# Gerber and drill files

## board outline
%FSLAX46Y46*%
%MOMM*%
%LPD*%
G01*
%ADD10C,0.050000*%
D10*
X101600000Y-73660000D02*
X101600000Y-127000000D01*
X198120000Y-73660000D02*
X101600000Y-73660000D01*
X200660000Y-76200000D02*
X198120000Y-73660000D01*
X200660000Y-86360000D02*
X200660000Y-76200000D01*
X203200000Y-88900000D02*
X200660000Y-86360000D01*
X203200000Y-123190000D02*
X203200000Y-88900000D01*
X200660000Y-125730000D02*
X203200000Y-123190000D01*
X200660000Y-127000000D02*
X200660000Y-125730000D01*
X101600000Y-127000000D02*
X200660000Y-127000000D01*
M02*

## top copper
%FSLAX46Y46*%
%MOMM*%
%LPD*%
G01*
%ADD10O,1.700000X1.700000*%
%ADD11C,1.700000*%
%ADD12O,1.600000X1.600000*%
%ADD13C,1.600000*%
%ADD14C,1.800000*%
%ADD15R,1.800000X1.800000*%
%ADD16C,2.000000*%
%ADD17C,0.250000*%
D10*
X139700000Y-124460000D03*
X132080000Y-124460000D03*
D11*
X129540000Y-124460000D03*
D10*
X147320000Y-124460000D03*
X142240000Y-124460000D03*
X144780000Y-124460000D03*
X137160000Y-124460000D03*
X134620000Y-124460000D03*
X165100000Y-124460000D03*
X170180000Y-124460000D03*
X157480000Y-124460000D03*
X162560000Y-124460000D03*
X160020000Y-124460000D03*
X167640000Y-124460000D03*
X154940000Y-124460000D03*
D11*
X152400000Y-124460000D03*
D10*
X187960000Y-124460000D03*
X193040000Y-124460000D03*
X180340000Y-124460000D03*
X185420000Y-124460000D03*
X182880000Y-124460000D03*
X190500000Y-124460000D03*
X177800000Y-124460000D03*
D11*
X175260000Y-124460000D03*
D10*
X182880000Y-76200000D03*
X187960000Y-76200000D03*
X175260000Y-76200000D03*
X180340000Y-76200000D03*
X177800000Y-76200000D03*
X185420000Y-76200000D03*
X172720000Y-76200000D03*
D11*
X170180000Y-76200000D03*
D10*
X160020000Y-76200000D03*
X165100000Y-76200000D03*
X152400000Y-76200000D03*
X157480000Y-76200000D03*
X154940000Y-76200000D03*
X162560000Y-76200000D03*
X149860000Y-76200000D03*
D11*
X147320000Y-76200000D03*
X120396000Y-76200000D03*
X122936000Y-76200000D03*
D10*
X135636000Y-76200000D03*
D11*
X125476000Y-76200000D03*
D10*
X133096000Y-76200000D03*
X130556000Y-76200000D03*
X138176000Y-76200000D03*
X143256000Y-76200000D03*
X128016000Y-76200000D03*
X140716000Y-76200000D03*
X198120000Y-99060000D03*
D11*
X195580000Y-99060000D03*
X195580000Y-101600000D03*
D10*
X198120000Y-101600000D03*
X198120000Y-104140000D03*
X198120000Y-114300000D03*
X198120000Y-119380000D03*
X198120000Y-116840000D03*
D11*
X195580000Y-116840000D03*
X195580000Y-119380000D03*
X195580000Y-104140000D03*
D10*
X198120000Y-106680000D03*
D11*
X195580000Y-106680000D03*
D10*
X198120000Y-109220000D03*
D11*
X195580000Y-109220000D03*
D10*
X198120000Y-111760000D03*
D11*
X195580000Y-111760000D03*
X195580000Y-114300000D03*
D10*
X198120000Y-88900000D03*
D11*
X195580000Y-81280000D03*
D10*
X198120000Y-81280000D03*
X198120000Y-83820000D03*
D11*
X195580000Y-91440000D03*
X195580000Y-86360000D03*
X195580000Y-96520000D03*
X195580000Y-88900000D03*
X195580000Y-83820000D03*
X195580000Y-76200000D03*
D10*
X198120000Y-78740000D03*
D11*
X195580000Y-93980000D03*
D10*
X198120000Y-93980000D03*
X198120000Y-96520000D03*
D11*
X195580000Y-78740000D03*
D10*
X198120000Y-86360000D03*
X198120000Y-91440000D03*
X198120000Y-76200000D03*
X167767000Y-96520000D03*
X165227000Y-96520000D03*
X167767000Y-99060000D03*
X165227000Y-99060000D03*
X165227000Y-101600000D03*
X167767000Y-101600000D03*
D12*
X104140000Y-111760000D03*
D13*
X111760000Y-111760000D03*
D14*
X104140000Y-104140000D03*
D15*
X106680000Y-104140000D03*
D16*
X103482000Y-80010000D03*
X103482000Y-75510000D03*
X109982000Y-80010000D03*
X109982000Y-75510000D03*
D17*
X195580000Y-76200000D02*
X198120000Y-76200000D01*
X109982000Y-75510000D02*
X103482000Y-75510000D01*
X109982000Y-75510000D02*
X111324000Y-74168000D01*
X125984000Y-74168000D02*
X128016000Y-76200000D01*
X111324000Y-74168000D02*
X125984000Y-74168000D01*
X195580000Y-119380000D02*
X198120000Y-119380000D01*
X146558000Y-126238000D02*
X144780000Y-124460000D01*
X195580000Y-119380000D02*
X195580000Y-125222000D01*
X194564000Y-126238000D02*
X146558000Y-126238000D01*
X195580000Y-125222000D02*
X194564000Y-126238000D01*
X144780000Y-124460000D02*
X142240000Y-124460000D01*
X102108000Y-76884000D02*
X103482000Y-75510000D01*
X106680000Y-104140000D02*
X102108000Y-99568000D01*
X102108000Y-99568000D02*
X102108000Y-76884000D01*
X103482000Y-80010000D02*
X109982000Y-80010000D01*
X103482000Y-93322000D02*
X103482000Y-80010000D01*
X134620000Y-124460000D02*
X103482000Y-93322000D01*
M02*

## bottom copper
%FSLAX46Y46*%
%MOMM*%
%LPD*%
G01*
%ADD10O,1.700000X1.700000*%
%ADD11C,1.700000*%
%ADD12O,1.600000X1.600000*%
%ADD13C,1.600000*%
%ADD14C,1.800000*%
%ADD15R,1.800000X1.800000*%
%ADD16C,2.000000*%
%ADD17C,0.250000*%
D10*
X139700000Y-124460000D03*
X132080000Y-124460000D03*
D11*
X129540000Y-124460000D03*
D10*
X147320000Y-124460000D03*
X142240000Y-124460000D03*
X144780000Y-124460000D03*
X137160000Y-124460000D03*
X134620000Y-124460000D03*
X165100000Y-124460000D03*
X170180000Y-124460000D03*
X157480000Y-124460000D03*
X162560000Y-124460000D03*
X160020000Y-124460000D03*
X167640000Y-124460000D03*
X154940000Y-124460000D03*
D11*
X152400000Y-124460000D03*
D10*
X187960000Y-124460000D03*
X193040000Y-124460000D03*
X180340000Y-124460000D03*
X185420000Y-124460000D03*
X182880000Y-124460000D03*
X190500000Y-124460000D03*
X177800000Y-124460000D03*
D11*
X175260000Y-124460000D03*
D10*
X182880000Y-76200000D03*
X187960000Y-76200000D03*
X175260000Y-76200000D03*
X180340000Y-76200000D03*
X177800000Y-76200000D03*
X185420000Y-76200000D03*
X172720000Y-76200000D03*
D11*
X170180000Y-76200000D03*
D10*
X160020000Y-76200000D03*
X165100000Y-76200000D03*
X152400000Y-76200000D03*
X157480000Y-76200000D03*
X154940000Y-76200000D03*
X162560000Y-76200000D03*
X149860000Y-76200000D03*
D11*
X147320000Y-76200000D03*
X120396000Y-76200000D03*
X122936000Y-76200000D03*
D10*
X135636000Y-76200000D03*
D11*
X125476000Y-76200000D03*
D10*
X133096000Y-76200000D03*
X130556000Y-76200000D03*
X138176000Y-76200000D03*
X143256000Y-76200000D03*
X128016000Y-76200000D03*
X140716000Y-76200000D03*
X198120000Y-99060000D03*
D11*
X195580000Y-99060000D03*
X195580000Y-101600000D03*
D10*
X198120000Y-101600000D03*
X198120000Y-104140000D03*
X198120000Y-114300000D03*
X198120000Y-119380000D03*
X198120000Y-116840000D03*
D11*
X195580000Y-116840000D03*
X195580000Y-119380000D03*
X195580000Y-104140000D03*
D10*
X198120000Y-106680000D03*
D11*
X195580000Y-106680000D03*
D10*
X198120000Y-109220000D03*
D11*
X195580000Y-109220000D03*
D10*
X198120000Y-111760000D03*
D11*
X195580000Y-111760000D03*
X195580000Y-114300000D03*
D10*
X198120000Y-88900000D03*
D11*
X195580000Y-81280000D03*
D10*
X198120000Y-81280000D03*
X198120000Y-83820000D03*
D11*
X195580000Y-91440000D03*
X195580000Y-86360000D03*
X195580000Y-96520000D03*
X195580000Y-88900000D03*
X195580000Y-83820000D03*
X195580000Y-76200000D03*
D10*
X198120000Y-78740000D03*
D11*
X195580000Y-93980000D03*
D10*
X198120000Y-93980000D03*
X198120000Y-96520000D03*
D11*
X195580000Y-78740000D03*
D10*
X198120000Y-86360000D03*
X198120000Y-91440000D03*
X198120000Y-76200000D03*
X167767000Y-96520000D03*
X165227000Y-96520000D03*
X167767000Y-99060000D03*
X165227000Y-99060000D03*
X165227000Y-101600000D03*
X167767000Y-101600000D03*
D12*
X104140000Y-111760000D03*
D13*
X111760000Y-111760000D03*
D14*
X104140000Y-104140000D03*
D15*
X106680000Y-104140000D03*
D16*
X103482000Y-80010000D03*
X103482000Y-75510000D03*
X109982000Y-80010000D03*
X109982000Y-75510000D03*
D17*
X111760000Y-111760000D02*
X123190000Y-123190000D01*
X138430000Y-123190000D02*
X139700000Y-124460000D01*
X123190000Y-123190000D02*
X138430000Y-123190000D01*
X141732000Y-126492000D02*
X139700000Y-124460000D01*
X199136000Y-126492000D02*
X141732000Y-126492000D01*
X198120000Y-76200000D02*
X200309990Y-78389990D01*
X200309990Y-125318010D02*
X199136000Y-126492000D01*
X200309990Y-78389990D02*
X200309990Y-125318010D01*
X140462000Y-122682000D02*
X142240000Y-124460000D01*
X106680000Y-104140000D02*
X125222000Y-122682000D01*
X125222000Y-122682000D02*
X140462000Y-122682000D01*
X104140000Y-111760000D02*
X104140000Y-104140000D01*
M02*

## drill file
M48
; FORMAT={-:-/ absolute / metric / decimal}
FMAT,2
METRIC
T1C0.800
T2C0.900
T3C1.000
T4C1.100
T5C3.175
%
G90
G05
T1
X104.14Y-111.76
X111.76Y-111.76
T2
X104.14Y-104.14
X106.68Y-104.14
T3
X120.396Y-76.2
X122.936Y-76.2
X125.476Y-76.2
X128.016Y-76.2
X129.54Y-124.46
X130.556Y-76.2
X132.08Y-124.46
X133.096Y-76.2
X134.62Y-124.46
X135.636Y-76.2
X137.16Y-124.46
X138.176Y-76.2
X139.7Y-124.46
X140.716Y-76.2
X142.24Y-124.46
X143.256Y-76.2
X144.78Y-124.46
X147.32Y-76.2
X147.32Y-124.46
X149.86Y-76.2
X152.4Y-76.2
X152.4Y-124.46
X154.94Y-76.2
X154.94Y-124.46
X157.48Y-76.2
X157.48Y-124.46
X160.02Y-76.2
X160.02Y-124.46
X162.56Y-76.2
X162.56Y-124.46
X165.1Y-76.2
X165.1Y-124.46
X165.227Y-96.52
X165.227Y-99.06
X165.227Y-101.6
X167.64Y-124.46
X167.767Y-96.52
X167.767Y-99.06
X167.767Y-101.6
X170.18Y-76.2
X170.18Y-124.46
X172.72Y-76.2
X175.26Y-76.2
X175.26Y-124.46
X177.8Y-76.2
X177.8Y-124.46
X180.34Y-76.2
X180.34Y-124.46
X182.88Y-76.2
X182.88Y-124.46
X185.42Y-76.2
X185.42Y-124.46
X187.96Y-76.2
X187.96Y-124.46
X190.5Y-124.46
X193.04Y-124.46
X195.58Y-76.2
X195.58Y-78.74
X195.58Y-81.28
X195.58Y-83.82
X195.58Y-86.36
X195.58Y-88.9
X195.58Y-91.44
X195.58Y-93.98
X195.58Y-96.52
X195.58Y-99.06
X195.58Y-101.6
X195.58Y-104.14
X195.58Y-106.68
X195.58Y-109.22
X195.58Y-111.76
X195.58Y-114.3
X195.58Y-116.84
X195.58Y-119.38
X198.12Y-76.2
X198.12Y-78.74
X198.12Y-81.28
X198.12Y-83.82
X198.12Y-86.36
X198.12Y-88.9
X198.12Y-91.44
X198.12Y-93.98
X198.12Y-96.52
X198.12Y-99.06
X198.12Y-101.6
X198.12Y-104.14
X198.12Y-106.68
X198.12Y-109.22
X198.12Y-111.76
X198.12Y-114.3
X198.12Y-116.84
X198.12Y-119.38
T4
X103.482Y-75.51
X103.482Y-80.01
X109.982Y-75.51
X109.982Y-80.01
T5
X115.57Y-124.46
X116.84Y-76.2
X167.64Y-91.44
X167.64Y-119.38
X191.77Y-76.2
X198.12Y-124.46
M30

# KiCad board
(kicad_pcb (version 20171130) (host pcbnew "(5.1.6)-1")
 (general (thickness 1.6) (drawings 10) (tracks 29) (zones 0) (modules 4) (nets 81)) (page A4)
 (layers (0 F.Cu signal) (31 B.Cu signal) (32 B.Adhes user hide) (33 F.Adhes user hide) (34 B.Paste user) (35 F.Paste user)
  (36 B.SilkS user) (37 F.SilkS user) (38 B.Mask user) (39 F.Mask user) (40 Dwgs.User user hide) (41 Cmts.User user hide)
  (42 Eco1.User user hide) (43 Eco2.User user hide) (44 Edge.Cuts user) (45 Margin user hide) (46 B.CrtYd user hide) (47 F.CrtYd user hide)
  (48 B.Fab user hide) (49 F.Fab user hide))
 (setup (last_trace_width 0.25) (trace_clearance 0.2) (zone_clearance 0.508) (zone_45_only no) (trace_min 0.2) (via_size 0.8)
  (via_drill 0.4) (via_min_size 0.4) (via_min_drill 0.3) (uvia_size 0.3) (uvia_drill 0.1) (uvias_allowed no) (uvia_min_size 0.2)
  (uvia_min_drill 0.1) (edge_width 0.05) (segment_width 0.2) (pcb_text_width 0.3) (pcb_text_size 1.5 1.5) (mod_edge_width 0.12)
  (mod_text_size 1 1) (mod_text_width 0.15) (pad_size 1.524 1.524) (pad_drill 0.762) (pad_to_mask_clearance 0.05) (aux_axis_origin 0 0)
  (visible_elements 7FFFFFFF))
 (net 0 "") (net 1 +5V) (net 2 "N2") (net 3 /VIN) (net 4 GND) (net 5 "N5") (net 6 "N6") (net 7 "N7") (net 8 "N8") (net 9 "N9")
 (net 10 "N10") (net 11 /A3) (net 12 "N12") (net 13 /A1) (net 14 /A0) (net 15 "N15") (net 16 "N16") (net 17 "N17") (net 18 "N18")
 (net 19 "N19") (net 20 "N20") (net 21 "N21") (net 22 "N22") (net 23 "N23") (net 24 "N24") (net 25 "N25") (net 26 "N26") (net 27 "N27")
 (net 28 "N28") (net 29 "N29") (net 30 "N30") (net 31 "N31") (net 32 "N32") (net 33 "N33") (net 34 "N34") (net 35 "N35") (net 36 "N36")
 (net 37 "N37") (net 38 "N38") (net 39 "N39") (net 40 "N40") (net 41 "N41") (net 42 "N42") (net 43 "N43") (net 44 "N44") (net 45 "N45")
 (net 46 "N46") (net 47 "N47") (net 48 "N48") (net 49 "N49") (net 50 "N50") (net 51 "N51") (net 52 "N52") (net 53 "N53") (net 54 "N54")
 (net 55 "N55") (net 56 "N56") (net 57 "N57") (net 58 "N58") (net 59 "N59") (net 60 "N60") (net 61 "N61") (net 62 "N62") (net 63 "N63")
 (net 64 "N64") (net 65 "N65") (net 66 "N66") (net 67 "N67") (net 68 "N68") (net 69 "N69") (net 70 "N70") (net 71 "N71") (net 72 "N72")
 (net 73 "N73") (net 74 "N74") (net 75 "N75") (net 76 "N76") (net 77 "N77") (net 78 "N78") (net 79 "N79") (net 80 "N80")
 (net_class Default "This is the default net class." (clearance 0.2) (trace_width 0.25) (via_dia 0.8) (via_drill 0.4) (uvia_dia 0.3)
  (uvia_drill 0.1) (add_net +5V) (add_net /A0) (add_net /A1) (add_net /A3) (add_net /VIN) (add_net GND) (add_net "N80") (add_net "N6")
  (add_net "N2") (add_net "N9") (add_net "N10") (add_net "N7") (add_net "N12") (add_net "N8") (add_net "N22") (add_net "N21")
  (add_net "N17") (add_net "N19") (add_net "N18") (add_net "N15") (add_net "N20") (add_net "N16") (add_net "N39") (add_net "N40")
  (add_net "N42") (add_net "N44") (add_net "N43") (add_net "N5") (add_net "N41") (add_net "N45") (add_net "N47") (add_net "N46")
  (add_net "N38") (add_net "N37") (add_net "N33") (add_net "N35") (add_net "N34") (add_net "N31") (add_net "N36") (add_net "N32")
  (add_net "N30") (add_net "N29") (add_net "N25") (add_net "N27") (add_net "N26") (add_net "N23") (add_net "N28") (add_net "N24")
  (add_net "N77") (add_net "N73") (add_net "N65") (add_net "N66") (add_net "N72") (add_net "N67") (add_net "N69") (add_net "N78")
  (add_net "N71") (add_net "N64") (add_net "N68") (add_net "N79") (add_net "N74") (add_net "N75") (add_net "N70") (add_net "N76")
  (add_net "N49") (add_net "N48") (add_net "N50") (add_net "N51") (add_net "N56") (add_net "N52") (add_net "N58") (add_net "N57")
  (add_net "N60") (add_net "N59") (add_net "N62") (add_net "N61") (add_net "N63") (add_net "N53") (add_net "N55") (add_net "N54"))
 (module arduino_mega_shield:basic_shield (layer F.Cu) (at 101.6 127)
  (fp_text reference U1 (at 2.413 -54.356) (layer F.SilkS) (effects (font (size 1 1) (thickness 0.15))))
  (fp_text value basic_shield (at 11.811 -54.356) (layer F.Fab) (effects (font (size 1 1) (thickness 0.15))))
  (pad 4 thru_hole oval (at 38.1 -2.54 90) (size 1.7 1.7) (drill 1) (layers *.Cu *.Mask) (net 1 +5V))
  (pad 1 thru_hole oval (at 30.48 -2.54 90) (size 1.7 1.7) (drill 1) (layers *.Cu *.Mask) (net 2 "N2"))
  (pad "" thru_hole circle (at 27.94 -2.54 90) (size 1.7 1.7) (drill 1) (layers *.Cu *.Mask))
  (pad 7 thru_hole oval (at 45.72 -2.54 90) (size 1.7 1.7) (drill 1) (layers *.Cu *.Mask) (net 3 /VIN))
  (pad 5 thru_hole oval (at 40.64 -2.54 90) (size 1.7 1.7) (drill 1) (layers *.Cu *.Mask) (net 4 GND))
  (pad 6 thru_hole oval (at 43.18 -2.54 90) (size 1.7 1.7) (drill 1) (layers *.Cu *.Mask) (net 4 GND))
  (pad 3 thru_hole oval (at 35.56 -2.54 90) (size 1.7 1.7) (drill 1) (layers *.Cu *.Mask) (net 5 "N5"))
  (pad 2 thru_hole oval (at 33.02 -2.54 90) (size 1.7 1.7) (drill 1) (layers *.Cu *.Mask B.SilkS) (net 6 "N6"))
  (pad 13 thru_hole oval (at 63.5 -2.54 90) (size 1.7 1.7) (drill 1) (layers *.Cu *.Mask) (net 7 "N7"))
  (pad 15 thru_hole oval (at 68.58 -2.54 90) (size 1.7 1.7) (drill 1) (layers *.Cu *.Mask) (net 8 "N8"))
  (pad 10 thru_hole oval (at 55.88 -2.54 90) (size 1.7 1.7) (drill 1) (layers *.Cu *.Mask) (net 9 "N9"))
  (pad 12 thru_hole oval (at 60.96 -2.54 90) (size 1.7 1.7) (drill 1) (layers *.Cu *.Mask) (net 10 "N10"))
  (pad 11 thru_hole oval (at 58.42 -2.54 90) (size 1.7 1.7) (drill 1) (layers *.Cu *.Mask) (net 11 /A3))
  (pad 14 thru_hole oval (at 66.04 -2.54 90) (size 1.7 1.7) (drill 1) (layers *.Cu *.Mask) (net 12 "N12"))
  (pad 9 thru_hole oval (at 53.34 -2.54 90) (size 1.7 1.7) (drill 1) (layers *.Cu *.Mask) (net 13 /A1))
  (pad 8 thru_hole circle (at 50.8 -2.54 90) (size 1.7 1.7) (drill 1) (layers *.Cu *.Mask) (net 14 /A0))
  (pad 21 thru_hole oval (at 86.36 -2.54 90) (size 1.7 1.7) (drill 1) (layers *.Cu *.Mask) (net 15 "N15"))
  (pad 23 thru_hole oval (at 91.44 -2.54 90) (size 1.7 1.7) (drill 1) (layers *.Cu *.Mask) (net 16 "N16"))
  (pad 18 thru_hole oval (at 78.74 -2.54 90) (size 1.7 1.7) (drill 1) (layers *.Cu *.Mask) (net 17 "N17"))
  (pad 20 thru_hole oval (at 83.82 -2.54 90) (size 1.7 1.7) (drill 1) (layers *.Cu *.Mask) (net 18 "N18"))
  (pad 19 thru_hole oval (at 81.28 -2.54 90) (size 1.7 1.7) (drill 1) (layers *.Cu *.Mask) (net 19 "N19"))
  (pad 22 thru_hole oval (at 88.9 -2.54 90) (size 1.7 1.7) (drill 1) (layers *.Cu *.Mask) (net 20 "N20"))
  (pad 17 thru_hole oval (at 76.2 -2.54 90) (size 1.7 1.7) (drill 1) (layers *.Cu *.Mask) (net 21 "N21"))
  (pad 16 thru_hole circle (at 73.66 -2.54 90) (size 1.7 1.7) (drill 1) (layers *.Cu *.Mask) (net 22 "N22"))
  (pad 47 thru_hole oval (at 81.28 -50.8 90) (size 1.7 1.7) (drill 1) (layers *.Cu *.Mask) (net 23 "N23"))
  (pad 49 thru_hole oval (at 86.36 -50.8 90) (size 1.7 1.7) (drill 1) (layers *.Cu *.Mask) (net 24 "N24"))
  (pad 44 thru_hole oval (at 73.66 -50.8 90) (size 1.7 1.7) (drill 1) (layers *.Cu *.Mask) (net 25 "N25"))
  (pad 46 thru_hole oval (at 78.74 -50.8 90) (size 1.7 1.7) (drill 1) (layers *.Cu *.Mask) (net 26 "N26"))
  (pad 45 thru_hole oval (at 76.2 -50.8 90) (size 1.7 1.7) (drill 1) (layers *.Cu *.Mask) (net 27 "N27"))
  (pad 48 thru_hole oval (at 83.82 -50.8 90) (size 1.7 1.7) (drill 1) (layers *.Cu *.Mask) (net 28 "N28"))
  (pad 43 thru_hole oval (at 71.12 -50.8 90) (size 1.7 1.7) (drill 1) (layers *.Cu *.Mask) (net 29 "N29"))
  (pad 42 thru_hole circle (at 68.58 -50.8 90) (size 1.7 1.7) (drill 1) (layers *.Cu *.Mask) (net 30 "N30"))
  (pad 39 thru_hole oval (at 58.42 -50.8 90) (size 1.7 1.7) (drill 1) (layers *.Cu *.Mask) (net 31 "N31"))
  (pad 41 thru_hole oval (at 63.5 -50.8 90) (size 1.7 1.7) (drill 1) (layers *.Cu *.Mask) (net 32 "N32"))
  (pad 36 thru_hole oval (at 50.8 -50.8 90) (size 1.7 1.7) (drill 1) (layers *.Cu *.Mask) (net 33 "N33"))
  (pad 38 thru_hole oval (at 55.88 -50.8 90) (size 1.7 1.7) (drill 1) (layers *.Cu *.Mask) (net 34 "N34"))
  (pad 37 thru_hole oval (at 53.34 -50.8 90) (size 1.7 1.7) (drill 1) (layers *.Cu *.Mask) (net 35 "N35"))
  (pad 40 thru_hole oval (at 60.96 -50.8 90) (size 1.7 1.7) (drill 1) (layers *.Cu *.Mask) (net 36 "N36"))
  (pad 35 thru_hole oval (at 48.26 -50.8 90) (size 1.7 1.7) (drill 1) (layers *.Cu *.Mask B.Paste) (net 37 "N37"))
  (pad 34 thru_hole circle (at 45.72 -50.8 90) (size 1.7 1.7) (drill 1) (layers *.Cu *.Mask) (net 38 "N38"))
  (pad 24 thru_hole circle (at 18.796 -50.8 90) (size 1.7 1.7) (drill 1) (layers *.Cu *.Mask) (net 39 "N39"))
  (pad 25 thru_hole circle (at 21.336 -50.8 90) (size 1.7 1.7) (drill 1) (layers *.Cu *.Mask) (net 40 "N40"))
  (pad 30 thru_hole oval (at 34.036 -50.8 90) (size 1.7 1.7) (drill 1) (layers *.Cu *.Mask) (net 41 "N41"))
  (pad 26 thru_hole circle (at 23.876 -50.8 90) (size 1.7 1.7) (drill 1) (layers *.Cu *.Mask) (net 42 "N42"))
  (pad 29 thru_hole oval (at 31.496 -50.8 90) (size 1.7 1.7) (drill 1) (layers *.Cu *.Mask) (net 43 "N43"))
  (pad 28 thru_hole oval (at 28.956 -50.8 90) (size 1.7 1.7) (drill 1) (layers *.Cu *.Mask) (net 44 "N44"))
  (pad 31 thru_hole oval (at 36.576 -50.8 90) (size 1.7 1.7) (drill 1) (layers *.Cu *.Mask) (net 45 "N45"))
  (pad 33 thru_hole oval (at 41.656 -50.8 90) (size 1.7 1.7) (drill 1) (layers *.Cu *.Mask) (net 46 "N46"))
  (pad 27 thru_hole oval (at 26.416 -50.8 90) (size 1.7 1.7) (drill 1) (layers *.Cu *.Mask) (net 4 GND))
  (pad 32 thru_hole oval (at 39.116 -50.8 90) (size 1.7 1.7) (drill 1) (layers *.Cu *.Mask) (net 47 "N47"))
  (pad 69 thru_hole oval (at 96.52 -27.94 90) (size 1.7 1.7) (drill 1) (layers *.Cu *.Mask) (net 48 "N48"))
  (pad 68 thru_hole circle (at 93.98 -27.94 90) (size 1.7 1.7) (drill 1) (layers *.Cu *.Mask) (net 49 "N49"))
  (pad 70 thru_hole circle (at 93.98 -25.4 90) (size 1.7 1.7) (drill 1) (layers *.Cu *.Mask) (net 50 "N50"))
  (pad 71 thru_hole oval (at 96.52 -25.4 90) (size 1.7 1.7) (drill 1) (layers *.Cu *.Mask) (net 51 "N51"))
  (pad 73 thru_hole oval (at 96.52 -22.86 90) (size 1.7 1.7) (drill 1) (layers *.Cu *.Mask) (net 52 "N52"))
  (pad 81 thru_hole oval (at 96.52 -12.7 90) (size 1.7 1.7) (drill 1) (layers *.Cu *.Mask) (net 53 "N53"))
  (pad 85 thru_hole oval (at 96.52 -7.62 90) (size 1.7 1.7) (drill 1) (layers *.Cu *.Mask) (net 4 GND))
  (pad 83 thru_hole oval (at 96.52 -10.16 90) (size 1.7 1.7) (drill 1) (layers *.Cu *.Mask) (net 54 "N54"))
  (pad 82 thru_hole circle (at 93.98 -10.16 90) (size 1.7 1.7) (drill 1) (layers *.Cu *.Mask) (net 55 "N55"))
  (pad 84 thru_hole circle (at 93.98 -7.62 90) (size 1.7 1.7) (drill 1) (layers *.Cu *.Mask) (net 4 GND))
  (pad 72 thru_hole circle (at 93.98 -22.86 90) (size 1.7 1.7) (drill 1) (layers *.Cu *.Mask) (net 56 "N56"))
  (pad 75 thru_hole oval (at 96.52 -20.32 90) (size 1.7 1.7) (drill 1) (layers *.Cu *.Mask) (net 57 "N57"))
  (pad 74 thru_hole circle (at 93.98 -20.32 90) (size 1.7 1.7) (drill 1) (layers *.Cu *.Mask) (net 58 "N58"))
  (pad 77 thru_hole oval (at 96.52 -17.78 90) (size 1.7 1.7) (drill 1) (layers *.Cu *.Mask) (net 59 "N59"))
  (pad 76 thru_hole circle (at 93.98 -17.78 90) (size 1.7 1.7) (drill 1) (layers *.Cu *.Mask) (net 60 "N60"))
  (pad 79 thru_hole oval (at 96.52 -15.24 90) (size 1.7 1.7) (drill 1) (layers *.Cu *.Mask) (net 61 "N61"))
  (pad 78 thru_hole circle (at 93.98 -15.24 90) (size 1.7 1.7) (drill 1) (layers *.Cu *.Mask) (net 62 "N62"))
  (pad 80 thru_hole circle (at 93.98 -12.7 90) (size 1.7 1.7) (drill 1) (layers *.Cu *.Mask) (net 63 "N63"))
  (pad 61 thru_hole oval (at 96.52 -38.1 90) (size 1.7 1.7) (drill 1) (layers *.Cu *.Mask) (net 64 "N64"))
  (pad 54 thru_hole circle (at 93.98 -45.72 90) (size 1.7 1.7) (drill 1) (layers *.Cu *.Mask) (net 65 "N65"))
  (pad 55 thru_hole oval (at 96.52 -45.72 90) (size 1.7 1.7) (drill 1) (layers *.Cu *.Mask) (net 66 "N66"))
  (pad 57 thru_hole oval (at 96.52 -43.18 90) (size 1.7 1.7) (drill 1) (layers *.Cu *.Mask) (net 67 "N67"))
  (pad 62 thru_hole circle (at 93.98 -35.56 90) (size 1.7 1.7) (drill 1) (layers *.Cu *.Mask) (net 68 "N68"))
  (pad 58 thru_hole circle (at 93.98 -40.64 90) (size 1.7 1.7) (drill 1) (layers *.Cu *.Mask) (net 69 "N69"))
  (pad 66 thru_hole circle (at 93.98 -30.48 90) (size 1.7 1.7) (drill 1) (layers *.Cu *.Mask) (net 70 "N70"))
  (pad 60 thru_hole circle (at 93.98 -38.1 90) (size 1.7 1.7) (drill 1) (layers *.Cu *.Mask) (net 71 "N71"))
  (pad 56 thru_hole circle (at 93.98 -43.18 90) (size 1.7 1.7) (drill 1) (layers *.Cu *.Mask) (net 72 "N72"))
  (pad 50 thru_hole circle (at 93.98 -50.8 90) (size 1.7 1.7) (drill 1) (layers *.Cu *.Mask) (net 1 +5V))
  (pad 53 thru_hole oval (at 96.52 -48.26 90) (size 1.7 1.7) (drill 1) (layers *.Cu *.Mask) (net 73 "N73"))
  (pad 64 thru_hole circle (at 93.98 -33.02 90) (size 1.7 1.7) (drill 1) (layers *.Cu *.Mask) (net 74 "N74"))
  (pad 65 thru_hole oval (at 96.52 -33.02 90) (size 1.7 1.7) (drill 1) (layers *.Cu *.Mask) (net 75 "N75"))
  (pad 67 thru_hole oval (at 96.52 -30.48 90) (size 1.7 1.7) (drill 1) (layers *.Cu *.Mask) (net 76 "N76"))
  (pad 52 thru_hole circle (at 93.98 -48.26 90) (size 1.7 1.7) (drill 1) (layers *.Cu *.Mask) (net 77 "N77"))
  (pad 59 thru_hole oval (at 96.52 -40.64 90) (size 1.7 1.7) (drill 1) (layers *.Cu *.Mask) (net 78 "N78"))
  (pad 63 thru_hole oval (at 96.52 -35.56 90) (size 1.7 1.7) (drill 1) (layers *.Cu *.Mask) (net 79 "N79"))
  (pad 51 thru_hole oval (at 96.52 -50.8 90) (size 1.7 1.7) (drill 1) (layers *.Cu *.Mask) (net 1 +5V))
  (pad "" np_thru_hole circle (at 13.97 -2.54 90) (size 3.175 3.175) (drill 3.175) (layers *.Cu *.Mask))
  (pad "" np_thru_hole circle (at 66.04 -7.62 90) (size 3.175 3.175) (drill 3.175) (layers *.Cu *.Mask))
  (pad "" np_thru_hole circle (at 66.04 -35.56 90) (size 3.175 3.175) (drill 3.175) (layers *.Cu *.Mask))
  (pad "" np_thru_hole circle (at 96.52 -2.54 90) (size 3.175 3.175) (drill 3.175) (layers *.Cu *.Mask))
  (pad "" np_thru_hole circle (at 90.17 -50.8 90) (size 3.175 3.175) (drill 3.175) (layers *.Cu *.Mask))
  (pad "" np_thru_hole circle (at 15.24 -50.8 90) (size 3.175 3.175) (drill 3.175) (layers *.Cu *.Mask))
  (pad "" thru_hole oval (at 66.167 -30.48 90) (size 1.7 1.7) (drill 1) (layers *.Cu *.Mask))
  (pad "" thru_hole oval (at 63.627 -30.48 90) (size 1.7 1.7) (drill 1) (layers *.Cu *.Mask))
  (pad "" thru_hole oval (at 66.167 -27.94 90) (size 1.7 1.7) (drill 1) (layers *.Cu *.Mask))
  (pad "" thru_hole oval (at 63.627 -27.94 90) (size 1.7 1.7) (drill 1) (layers *.Cu *.Mask))
  (pad "" thru_hole oval (at 63.627 -25.4 90) (size 1.7 1.7) (drill 1) (layers *.Cu *.Mask))
  (pad "" thru_hole oval (at 66.167 -25.4 90) (size 1.7 1.7) (drill 1) (layers *.Cu *.Mask)))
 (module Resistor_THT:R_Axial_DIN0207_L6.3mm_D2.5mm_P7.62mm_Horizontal (layer F.Cu) (at 111.76 111.76 180)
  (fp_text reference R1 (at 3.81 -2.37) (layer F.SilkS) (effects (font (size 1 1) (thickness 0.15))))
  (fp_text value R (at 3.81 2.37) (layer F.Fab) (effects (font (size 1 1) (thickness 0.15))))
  (pad 2 thru_hole oval (at 7.62 0 180) (size 1.6 1.6) (drill 0.8) (layers *.Cu *.Mask) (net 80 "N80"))
  (pad 1 thru_hole circle (at 0 0 180) (size 1.6 1.6) (drill 0.8) (layers *.Cu *.Mask) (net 1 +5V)))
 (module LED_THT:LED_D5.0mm (layer F.Cu) (at 106.68 104.14 180)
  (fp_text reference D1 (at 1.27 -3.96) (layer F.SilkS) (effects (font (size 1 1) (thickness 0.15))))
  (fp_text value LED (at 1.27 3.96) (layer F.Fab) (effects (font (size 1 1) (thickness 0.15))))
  (pad 2 thru_hole circle (at 2.54 0 180) (size 1.8 1.8) (drill 0.9) (layers *.Cu *.Mask) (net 80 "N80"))
  (pad 1 thru_hole rect (at 0 0 180) (size 1.8 1.8) (drill 0.9) (layers *.Cu *.Mask) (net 4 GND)))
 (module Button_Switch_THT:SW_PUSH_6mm (layer F.Cu) (at 109.982 80.01 180)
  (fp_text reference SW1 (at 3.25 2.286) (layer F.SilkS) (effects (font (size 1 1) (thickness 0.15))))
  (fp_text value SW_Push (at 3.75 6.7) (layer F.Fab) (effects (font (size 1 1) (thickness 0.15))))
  (pad 1 thru_hole circle (at 6.5 0 270) (size 2 2) (drill 1.1) (layers *.Cu *.Mask) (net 6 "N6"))
  (pad 2 thru_hole circle (at 6.5 4.5 270) (size 2 2) (drill 1.1) (layers *.Cu *.Mask) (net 4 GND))
  (pad 1 thru_hole circle (at 0 0 270) (size 2 2) (drill 1.1) (layers *.Cu *.Mask) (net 6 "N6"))
  (pad 2 thru_hole circle (at 0 4.5 270) (size 2 2) (drill 1.1) (layers *.Cu *.Mask) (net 4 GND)))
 (gr_line (start 101.6 73.66) (end 101.6 127) (layer Edge.Cuts) (width 0.05))
 (gr_line (start 198.12 73.66) (end 101.6 73.66) (layer Edge.Cuts) (width 0.05))
 (gr_line (start 200.66 76.2) (end 198.12 73.66) (layer Edge.Cuts) (width 0.05))
 (gr_line (start 200.66 86.36) (end 200.66 76.2) (layer Edge.Cuts) (width 0.05))
 (gr_line (start 203.2 88.9) (end 200.66 86.36) (layer Edge.Cuts) (width 0.05))
 (gr_line (start 203.2 123.19) (end 203.2 88.9) (layer Edge.Cuts) (width 0.05))
 (gr_line (start 200.66 125.73) (end 203.2 123.19) (layer Edge.Cuts) (width 0.05))
 (gr_line (start 200.66 127) (end 200.66 125.73) (layer Edge.Cuts) (width 0.05))
 (gr_line (start 101.6 127) (end 200.66 127) (layer Edge.Cuts) (width 0.05))
 (segment (start 111.76 111.76) (end 123.19 123.19) (width 0.25) (layer B.Cu) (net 1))
 (segment (start 138.43 123.19) (end 139.7 124.46) (width 0.25) (layer B.Cu) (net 1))
 (segment (start 123.19 123.19) (end 138.43 123.19) (width 0.25) (layer B.Cu) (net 1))
 (segment (start 195.58 76.2) (end 198.12 76.2) (width 0.25) (layer F.Cu) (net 1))
 (segment (start 141.732 126.492) (end 139.7 124.46) (width 0.25) (layer B.Cu) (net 1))
 (segment (start 199.136 126.492) (end 141.732 126.492) (width 0.25) (layer B.Cu) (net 1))
 (segment (start 198.12 76.2) (end 200.30999 78.38999) (width 0.25) (layer B.Cu) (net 1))
 (segment (start 200.30999 125.31801) (end 199.136 126.492) (width 0.25) (layer B.Cu) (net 1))
 (segment (start 200.30999 78.38999) (end 200.30999 125.31801) (width 0.25) (layer B.Cu) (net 1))
 (segment (start 109.982 75.51) (end 103.482 75.51) (width 0.25) (layer F.Cu) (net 4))
 (segment (start 140.462 122.682) (end 142.24 124.46) (width 0.25) (layer B.Cu) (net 4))
 (segment (start 106.68 104.14) (end 125.222 122.682) (width 0.25) (layer B.Cu) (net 4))
 (segment (start 125.222 122.682) (end 140.462 122.682) (width 0.25) (layer B.Cu) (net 4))
 (segment (start 109.982 75.51) (end 111.324 74.168) (width 0.25) (layer F.Cu) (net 4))
 (segment (start 125.984 74.168) (end 128.016 76.2) (width 0.25) (layer F.Cu) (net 4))
 (segment (start 111.324 74.168) (end 125.984 74.168) (width 0.25) (layer F.Cu) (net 4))
 (segment (start 195.58 119.38) (end 198.12 119.38) (width 0.25) (layer F.Cu) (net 4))
 (segment (start 146.558 126.238) (end 144.78 124.46) (width 0.25) (layer F.Cu) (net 4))
 (segment (start 195.58 119.38) (end 195.58 125.222) (width 0.25) (layer F.Cu) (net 4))
 (segment (start 194.564 126.238) (end 146.558 126.238) (width 0.25) (layer F.Cu) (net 4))
 (segment (start 195.58 125.222) (end 194.564 126.238) (width 0.25) (layer F.Cu) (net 4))
 (segment (start 144.78 124.46) (end 142.24 124.46) (width 0.25) (layer F.Cu) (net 4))
 (segment (start 102.108 76.884) (end 103.482 75.51) (width 0.25) (layer F.Cu) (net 4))
 (segment (start 106.68 104.14) (end 102.108 99.568) (width 0.25) (layer F.Cu) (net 4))
 (segment (start 102.108 99.568) (end 102.108 76.884) (width 0.25) (layer F.Cu) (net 4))
 (segment (start 103.482 80.01) (end 109.982 80.01) (width 0.25) (layer F.Cu) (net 6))
 (segment (start 103.482 93.322) (end 103.482 80.01) (width 0.25) (layer F.Cu) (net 6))
 (segment (start 134.62 124.46) (end 103.482 93.322) (width 0.25) (layer F.Cu) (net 6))
 (segment (start 104.14 111.76) (end 104.14 104.14) (width 0.25) (layer B.Cu) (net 80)))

